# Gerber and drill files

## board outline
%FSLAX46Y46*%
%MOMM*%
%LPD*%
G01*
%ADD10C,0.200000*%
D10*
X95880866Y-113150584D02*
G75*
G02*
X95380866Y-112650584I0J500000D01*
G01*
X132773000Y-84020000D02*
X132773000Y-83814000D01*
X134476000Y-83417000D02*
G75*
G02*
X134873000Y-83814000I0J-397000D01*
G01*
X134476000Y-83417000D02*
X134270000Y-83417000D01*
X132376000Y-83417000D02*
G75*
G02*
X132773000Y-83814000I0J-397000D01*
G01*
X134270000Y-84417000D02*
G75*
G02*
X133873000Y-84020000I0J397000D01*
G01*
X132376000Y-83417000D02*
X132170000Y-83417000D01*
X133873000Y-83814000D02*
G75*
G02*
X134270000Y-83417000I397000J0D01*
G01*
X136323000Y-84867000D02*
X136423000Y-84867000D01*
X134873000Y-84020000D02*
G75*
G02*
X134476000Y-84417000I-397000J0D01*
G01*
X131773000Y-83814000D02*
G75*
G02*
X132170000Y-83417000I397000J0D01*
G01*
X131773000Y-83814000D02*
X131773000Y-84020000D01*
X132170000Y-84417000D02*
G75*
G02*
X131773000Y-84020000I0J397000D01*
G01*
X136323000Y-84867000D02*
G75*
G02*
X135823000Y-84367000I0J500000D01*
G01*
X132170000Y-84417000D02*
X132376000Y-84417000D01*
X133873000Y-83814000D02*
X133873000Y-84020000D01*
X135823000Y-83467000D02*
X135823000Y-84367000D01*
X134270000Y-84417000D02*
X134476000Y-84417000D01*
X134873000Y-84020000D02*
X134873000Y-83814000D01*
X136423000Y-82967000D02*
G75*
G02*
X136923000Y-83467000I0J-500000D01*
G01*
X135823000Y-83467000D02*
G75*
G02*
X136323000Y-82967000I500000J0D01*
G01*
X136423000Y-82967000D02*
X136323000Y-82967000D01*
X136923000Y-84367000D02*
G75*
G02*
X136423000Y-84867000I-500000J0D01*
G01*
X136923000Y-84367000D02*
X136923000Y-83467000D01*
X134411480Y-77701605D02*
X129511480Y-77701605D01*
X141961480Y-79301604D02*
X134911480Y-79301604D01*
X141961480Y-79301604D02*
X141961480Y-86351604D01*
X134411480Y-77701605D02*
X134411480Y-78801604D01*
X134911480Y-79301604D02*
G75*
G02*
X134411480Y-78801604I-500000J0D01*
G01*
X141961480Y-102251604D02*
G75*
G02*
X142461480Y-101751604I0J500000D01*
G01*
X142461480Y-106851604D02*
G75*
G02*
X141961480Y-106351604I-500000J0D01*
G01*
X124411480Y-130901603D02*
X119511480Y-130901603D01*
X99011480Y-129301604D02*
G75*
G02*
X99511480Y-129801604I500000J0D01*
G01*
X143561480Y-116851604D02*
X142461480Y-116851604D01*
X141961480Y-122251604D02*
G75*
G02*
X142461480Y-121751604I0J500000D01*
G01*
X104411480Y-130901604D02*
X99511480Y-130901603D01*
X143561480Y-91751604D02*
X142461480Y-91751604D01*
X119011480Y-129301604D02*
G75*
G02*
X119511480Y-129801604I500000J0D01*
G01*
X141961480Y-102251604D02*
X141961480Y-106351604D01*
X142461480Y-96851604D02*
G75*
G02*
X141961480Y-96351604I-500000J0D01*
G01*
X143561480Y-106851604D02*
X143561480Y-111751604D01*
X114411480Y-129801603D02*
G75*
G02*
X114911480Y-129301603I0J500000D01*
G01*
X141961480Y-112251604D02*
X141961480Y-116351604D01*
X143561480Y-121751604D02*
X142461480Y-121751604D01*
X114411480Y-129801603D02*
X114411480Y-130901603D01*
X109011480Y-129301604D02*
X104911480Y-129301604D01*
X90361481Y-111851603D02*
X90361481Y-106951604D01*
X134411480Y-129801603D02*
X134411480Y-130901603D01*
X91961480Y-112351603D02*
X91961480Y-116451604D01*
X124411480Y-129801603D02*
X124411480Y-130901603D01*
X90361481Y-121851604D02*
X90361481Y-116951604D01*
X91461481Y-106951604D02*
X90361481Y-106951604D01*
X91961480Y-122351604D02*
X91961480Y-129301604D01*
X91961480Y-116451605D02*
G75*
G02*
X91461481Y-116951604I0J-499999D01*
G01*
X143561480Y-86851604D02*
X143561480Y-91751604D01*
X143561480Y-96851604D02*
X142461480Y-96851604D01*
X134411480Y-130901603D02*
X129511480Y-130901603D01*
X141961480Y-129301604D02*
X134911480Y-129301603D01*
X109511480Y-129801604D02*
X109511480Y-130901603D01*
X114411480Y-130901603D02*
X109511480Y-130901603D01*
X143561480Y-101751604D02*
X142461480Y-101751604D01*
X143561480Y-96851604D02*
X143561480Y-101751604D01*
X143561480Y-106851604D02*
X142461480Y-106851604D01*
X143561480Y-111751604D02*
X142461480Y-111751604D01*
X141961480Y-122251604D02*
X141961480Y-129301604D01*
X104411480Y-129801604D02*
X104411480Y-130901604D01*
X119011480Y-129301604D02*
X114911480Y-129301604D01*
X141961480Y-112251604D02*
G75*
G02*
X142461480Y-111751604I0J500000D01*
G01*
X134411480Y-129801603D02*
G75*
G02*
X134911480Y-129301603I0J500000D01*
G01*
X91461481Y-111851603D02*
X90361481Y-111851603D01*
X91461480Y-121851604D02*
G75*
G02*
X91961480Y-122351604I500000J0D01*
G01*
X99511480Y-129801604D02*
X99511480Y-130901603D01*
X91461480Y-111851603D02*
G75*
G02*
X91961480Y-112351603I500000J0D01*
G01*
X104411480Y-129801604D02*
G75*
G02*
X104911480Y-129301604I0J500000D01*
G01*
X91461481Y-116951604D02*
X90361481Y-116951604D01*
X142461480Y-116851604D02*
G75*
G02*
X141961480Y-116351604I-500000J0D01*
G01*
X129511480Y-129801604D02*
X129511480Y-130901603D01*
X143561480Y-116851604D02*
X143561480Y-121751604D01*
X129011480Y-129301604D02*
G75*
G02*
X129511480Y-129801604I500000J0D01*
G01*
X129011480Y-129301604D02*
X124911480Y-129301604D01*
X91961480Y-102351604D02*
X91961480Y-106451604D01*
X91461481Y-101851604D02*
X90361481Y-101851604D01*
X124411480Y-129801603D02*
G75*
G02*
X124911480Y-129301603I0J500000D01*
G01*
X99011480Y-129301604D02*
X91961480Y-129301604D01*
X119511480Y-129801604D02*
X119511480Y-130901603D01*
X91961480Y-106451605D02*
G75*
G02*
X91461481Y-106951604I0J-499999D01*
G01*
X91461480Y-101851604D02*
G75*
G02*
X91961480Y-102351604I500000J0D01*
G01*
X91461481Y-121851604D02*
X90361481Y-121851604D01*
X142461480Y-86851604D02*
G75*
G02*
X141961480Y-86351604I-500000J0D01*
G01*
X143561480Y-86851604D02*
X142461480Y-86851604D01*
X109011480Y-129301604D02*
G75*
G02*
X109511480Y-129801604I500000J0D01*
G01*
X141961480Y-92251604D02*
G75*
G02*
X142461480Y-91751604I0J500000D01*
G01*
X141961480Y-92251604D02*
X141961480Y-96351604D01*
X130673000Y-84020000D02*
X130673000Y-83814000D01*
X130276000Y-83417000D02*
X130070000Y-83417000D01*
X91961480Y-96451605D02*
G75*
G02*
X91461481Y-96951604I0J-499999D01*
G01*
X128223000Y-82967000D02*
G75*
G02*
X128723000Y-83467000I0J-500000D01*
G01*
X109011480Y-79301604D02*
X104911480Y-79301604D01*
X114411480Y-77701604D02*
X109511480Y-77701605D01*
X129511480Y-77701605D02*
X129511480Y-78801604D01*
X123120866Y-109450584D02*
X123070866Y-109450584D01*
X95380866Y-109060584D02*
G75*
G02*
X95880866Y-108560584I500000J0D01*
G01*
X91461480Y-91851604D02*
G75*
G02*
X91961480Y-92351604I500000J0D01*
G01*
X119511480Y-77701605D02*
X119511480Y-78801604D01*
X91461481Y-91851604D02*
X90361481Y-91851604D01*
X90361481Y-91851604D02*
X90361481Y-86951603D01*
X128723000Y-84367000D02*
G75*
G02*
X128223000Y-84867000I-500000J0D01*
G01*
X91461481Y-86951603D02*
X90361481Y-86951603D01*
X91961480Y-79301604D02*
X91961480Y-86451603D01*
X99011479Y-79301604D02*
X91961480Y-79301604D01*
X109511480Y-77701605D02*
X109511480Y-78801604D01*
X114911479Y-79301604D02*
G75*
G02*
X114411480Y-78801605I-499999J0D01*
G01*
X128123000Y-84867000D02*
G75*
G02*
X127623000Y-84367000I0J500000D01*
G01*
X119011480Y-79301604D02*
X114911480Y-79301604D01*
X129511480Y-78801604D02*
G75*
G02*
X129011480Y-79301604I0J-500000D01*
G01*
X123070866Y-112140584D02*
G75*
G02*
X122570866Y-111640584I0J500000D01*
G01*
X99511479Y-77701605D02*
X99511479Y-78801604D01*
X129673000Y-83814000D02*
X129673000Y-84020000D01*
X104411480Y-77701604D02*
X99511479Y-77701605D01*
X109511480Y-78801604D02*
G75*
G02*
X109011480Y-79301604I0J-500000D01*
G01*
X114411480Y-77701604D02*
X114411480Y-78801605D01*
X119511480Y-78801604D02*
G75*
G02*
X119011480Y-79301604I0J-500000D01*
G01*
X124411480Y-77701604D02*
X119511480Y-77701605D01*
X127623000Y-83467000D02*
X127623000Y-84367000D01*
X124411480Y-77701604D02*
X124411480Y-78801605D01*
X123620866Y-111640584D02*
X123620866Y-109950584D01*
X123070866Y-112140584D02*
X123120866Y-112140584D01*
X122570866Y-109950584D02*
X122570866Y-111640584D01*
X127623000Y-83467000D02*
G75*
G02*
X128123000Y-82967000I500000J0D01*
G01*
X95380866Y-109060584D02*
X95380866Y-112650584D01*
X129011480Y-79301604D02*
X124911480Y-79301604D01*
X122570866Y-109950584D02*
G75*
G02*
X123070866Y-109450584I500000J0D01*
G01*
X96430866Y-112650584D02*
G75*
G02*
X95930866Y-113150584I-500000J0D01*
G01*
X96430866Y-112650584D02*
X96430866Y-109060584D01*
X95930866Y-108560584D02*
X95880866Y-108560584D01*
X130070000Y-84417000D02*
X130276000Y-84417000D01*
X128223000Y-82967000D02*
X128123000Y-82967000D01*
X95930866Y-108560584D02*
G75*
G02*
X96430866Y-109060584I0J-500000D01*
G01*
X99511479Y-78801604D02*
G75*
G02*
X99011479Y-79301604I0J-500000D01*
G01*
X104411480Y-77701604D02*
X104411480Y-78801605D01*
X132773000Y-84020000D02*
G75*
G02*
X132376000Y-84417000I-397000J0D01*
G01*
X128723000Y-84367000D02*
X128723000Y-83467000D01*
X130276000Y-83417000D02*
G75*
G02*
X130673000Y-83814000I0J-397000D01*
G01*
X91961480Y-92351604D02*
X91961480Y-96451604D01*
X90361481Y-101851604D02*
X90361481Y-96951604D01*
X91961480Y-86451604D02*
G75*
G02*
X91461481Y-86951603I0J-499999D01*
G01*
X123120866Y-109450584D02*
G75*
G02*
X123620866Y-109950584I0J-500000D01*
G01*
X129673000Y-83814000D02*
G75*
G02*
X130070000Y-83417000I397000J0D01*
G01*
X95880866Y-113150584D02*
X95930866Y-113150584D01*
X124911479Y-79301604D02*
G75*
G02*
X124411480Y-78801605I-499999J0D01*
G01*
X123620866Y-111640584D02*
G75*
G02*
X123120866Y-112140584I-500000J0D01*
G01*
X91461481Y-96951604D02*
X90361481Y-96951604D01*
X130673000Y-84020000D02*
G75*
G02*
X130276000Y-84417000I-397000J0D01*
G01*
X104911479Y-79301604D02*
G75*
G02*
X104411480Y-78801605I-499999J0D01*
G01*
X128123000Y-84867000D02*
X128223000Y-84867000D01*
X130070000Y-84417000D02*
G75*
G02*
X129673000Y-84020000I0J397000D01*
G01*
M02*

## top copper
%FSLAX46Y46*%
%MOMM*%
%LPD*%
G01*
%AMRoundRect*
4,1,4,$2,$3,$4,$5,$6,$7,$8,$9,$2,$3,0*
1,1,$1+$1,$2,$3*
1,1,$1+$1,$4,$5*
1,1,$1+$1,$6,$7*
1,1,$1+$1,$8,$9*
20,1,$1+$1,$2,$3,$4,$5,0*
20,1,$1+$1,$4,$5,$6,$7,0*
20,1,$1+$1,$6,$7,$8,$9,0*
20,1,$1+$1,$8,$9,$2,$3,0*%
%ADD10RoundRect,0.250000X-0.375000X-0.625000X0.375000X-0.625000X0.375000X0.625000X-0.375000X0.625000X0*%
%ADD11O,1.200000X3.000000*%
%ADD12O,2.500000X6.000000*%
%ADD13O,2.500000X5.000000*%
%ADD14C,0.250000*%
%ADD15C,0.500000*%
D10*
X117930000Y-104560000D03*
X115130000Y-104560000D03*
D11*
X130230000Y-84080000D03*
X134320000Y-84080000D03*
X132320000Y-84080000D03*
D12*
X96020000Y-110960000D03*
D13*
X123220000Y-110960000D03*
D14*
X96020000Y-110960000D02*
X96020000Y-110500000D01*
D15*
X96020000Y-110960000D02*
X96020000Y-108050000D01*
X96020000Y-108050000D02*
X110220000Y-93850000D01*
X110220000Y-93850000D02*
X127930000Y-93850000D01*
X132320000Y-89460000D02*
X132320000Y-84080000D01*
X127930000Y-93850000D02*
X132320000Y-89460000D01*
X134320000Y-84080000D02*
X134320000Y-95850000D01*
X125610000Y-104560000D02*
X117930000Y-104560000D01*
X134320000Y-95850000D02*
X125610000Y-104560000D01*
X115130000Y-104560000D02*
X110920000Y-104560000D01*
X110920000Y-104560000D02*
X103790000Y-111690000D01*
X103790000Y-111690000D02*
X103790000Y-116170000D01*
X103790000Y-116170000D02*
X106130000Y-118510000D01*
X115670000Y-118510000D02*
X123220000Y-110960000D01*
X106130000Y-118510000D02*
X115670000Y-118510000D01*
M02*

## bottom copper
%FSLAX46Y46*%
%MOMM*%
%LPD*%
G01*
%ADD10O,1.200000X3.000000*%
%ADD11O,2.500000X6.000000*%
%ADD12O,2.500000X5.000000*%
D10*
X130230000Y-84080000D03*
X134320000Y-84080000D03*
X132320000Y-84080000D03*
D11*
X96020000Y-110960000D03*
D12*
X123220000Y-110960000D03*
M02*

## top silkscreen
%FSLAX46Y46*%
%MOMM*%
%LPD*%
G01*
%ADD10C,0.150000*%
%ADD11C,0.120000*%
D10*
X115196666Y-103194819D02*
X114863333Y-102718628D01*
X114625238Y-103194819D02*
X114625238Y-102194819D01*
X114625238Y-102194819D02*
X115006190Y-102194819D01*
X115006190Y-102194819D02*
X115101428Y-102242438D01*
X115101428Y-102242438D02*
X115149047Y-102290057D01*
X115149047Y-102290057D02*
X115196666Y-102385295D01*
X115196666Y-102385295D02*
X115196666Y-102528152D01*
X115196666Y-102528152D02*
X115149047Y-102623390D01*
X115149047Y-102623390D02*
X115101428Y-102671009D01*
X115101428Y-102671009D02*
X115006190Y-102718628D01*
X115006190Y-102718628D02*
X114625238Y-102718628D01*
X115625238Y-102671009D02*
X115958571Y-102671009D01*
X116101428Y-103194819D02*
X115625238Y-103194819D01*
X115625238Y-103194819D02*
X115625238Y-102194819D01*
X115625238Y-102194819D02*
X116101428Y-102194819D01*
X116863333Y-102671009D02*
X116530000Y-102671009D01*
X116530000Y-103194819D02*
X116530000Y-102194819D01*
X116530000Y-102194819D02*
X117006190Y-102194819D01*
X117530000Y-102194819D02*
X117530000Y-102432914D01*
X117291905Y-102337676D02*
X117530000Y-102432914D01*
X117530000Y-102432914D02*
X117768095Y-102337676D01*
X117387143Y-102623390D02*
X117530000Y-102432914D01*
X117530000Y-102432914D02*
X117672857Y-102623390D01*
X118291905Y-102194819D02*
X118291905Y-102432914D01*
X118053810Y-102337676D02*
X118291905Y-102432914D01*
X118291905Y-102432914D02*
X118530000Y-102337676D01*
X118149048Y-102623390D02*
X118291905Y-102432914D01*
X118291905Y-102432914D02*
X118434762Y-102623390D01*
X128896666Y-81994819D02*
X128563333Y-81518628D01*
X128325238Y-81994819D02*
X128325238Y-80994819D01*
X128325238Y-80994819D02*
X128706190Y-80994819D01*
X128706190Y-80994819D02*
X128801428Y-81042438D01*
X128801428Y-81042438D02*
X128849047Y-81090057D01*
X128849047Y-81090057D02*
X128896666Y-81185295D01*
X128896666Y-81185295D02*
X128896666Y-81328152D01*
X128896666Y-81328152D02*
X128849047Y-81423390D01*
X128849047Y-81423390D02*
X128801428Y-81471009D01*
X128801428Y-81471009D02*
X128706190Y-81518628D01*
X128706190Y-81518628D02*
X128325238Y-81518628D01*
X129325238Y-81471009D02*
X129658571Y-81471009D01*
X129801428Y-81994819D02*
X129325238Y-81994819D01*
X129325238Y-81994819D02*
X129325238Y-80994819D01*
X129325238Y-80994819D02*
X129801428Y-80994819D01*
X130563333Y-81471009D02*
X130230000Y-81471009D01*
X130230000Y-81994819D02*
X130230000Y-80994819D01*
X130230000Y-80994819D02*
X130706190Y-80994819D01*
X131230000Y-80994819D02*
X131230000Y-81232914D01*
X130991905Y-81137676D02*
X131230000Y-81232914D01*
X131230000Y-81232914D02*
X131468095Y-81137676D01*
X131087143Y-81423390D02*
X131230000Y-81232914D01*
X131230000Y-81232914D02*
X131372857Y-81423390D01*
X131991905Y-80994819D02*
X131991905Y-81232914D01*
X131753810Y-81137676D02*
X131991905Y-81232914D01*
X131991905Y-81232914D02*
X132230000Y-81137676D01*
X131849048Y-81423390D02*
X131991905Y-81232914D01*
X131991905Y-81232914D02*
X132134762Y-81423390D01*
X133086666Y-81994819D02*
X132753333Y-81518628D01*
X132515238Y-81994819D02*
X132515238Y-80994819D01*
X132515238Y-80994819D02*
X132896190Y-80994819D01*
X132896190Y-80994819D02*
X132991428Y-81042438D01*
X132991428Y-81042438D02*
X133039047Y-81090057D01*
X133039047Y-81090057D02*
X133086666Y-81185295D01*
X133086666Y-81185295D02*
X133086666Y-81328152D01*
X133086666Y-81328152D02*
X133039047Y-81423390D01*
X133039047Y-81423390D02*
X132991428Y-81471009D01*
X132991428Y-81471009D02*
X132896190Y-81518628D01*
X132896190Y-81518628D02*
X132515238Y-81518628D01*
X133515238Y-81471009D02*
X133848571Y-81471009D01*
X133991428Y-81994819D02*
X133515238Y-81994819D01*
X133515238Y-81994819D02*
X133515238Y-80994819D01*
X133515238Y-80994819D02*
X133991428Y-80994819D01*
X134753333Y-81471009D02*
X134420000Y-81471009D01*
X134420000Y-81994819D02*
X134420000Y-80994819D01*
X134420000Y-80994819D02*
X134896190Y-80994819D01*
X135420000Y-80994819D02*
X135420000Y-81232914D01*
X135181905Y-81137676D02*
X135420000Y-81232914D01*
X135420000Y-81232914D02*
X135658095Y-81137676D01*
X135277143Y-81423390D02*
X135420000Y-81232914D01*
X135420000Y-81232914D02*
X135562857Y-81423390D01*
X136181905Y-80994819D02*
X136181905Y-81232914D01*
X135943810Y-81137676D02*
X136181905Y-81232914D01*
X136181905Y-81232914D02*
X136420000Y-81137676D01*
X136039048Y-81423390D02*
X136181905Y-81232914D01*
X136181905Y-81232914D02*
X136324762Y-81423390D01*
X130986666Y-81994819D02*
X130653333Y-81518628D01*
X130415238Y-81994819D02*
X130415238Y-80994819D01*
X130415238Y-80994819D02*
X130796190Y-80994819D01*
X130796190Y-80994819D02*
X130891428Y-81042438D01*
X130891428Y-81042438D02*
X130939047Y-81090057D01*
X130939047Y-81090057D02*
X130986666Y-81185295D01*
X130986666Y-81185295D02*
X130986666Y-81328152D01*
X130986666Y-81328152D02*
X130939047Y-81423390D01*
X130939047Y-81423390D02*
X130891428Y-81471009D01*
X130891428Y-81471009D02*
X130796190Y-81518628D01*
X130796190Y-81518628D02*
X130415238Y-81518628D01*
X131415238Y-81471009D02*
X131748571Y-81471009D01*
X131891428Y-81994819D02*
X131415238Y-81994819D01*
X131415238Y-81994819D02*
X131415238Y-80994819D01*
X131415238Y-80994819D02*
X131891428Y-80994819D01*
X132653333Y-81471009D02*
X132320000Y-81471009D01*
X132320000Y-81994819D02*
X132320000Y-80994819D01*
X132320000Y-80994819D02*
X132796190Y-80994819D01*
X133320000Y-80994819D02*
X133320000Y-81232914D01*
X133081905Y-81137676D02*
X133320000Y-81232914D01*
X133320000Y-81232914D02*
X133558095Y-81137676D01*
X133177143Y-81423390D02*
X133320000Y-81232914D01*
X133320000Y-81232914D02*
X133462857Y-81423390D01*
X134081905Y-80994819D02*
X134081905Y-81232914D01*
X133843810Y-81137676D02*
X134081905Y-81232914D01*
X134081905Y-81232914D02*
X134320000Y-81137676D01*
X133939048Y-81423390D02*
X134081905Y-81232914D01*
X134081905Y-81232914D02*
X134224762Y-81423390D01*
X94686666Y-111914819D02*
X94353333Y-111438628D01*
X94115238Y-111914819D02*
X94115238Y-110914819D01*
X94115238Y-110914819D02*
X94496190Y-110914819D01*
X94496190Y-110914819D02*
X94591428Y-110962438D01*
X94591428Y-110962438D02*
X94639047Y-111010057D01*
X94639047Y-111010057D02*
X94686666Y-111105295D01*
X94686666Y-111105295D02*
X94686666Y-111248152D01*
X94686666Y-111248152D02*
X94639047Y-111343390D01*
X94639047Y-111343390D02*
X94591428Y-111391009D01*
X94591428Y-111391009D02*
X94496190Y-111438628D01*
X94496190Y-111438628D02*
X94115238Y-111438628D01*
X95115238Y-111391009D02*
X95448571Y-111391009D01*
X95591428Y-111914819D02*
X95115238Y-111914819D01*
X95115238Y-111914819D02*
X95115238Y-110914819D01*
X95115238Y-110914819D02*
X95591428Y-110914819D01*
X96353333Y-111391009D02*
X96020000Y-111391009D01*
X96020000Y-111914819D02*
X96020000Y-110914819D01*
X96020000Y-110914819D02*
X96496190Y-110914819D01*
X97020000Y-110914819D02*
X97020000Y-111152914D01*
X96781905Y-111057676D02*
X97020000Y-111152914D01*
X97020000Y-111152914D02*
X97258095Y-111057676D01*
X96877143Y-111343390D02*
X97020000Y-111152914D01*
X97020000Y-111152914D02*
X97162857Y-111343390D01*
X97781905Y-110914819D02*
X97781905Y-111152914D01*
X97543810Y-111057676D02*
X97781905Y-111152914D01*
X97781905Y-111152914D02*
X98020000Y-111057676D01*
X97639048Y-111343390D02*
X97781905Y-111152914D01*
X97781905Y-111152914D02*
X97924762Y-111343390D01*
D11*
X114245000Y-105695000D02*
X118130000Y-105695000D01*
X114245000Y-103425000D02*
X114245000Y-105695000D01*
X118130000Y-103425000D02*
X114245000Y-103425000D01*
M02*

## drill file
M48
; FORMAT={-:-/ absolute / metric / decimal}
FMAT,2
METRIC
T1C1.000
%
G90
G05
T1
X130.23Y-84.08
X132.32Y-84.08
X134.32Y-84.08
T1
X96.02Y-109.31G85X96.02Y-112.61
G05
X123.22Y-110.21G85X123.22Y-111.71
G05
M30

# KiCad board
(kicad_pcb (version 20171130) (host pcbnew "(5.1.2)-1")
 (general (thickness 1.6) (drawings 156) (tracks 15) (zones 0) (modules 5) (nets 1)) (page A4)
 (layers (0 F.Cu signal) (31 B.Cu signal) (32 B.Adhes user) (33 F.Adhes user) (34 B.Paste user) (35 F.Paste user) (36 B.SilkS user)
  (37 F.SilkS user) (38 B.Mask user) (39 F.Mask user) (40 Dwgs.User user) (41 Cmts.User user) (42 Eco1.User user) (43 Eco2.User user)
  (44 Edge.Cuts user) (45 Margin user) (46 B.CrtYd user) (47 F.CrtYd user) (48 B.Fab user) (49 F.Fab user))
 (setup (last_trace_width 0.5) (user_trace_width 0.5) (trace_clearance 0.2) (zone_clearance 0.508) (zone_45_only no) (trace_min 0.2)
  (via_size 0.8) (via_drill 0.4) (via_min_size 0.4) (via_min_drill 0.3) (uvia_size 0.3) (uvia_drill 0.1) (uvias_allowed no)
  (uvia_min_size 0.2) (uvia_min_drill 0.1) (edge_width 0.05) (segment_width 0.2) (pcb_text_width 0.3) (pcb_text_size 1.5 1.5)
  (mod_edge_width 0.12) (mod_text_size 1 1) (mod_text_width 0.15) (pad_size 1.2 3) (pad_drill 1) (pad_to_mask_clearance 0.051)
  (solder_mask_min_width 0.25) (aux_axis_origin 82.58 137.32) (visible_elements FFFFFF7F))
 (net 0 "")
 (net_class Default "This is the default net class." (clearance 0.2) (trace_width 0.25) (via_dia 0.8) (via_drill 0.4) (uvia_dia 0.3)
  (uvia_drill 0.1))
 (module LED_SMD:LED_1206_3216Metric (layer F.Cu) (at 116.53 104.56)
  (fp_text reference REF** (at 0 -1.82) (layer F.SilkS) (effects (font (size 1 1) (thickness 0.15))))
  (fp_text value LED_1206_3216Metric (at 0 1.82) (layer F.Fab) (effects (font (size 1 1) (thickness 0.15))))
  (fp_line (start -2.285 1.135) (end 1.6 1.135) (layer F.SilkS) (width 0.12))
  (fp_line (start -2.285 -1.135) (end -2.285 1.135) (layer F.SilkS) (width 0.12))
  (fp_line (start 1.6 -1.135) (end -2.285 -1.135) (layer F.SilkS) (width 0.12))
  (pad 2 smd roundrect (at 1.4 0) (size 1.25 1.75) (layers F.Cu F.Paste F.Mask) (roundrect_rratio 0.2))
  (pad 1 smd roundrect (at -1.4 0) (size 1.25 1.75) (layers F.Cu F.Paste F.Mask) (roundrect_rratio 0.2)))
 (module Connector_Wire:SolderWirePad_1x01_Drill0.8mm (layer F.Cu) (at 130.23 84.08)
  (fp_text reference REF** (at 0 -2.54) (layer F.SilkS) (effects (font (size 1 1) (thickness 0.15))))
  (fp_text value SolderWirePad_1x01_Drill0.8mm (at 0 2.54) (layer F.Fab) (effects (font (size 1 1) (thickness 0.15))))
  (pad 1 thru_hole oval (at 0 0) (size 1.2 3) (drill 1) (layers F.Cu)))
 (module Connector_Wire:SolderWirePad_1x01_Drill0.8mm (layer F.Cu) (at 134.42 84.08)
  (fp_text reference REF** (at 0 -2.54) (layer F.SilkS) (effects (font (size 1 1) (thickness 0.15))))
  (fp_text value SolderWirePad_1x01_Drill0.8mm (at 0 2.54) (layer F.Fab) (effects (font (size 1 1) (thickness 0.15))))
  (pad 1 thru_hole oval (at -0.1 0) (size 1.2 3) (drill 1) (layers F.Cu)))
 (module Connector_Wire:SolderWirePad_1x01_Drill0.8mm (layer F.Cu) (at 132.32 84.08)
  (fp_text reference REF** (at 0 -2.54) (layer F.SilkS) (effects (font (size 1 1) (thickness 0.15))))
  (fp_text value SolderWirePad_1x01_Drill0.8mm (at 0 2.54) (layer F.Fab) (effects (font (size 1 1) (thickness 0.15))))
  (pad 1 thru_hole oval (at 0 0) (size 1.2 3) (drill 1) (layers F.Cu)))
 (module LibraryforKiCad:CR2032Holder (layer F.Cu) (at 96.02 110.96)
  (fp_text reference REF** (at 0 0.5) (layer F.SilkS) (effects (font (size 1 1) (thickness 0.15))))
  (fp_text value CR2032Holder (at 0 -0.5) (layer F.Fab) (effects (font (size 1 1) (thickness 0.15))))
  (pad 2 thru_hole oval (at 0 0) (size 2.5 6) (drill oval 1 4.3) (layers F.Cu F.Adhes))
  (pad 1 thru_hole oval (at 27.2 0) (size 2.5 5) (drill oval 1 2.5) (layers F.Cu)))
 (gr_arc (start 95.880866 112.650584) (end 95.380866 112.650584) (angle -90) (layer Edge.Cuts) (width 0.2))
 (gr_line (start 132.773 84.02) (end 132.773 83.814) (layer Edge.Cuts) (width 0.2))
 (gr_arc (start 134.476 83.814) (end 134.873 83.814) (angle -90) (layer Edge.Cuts) (width 0.2))
 (gr_line (start 134.476 83.417) (end 134.27 83.417) (layer Edge.Cuts) (width 0.2))
 (gr_arc (start 132.376 83.814) (end 132.773 83.814) (angle -90) (layer Edge.Cuts) (width 0.2))
 (gr_arc (start 134.27 84.02) (end 133.873 84.02) (angle -90) (layer Edge.Cuts) (width 0.2))
 (gr_line (start 132.376 83.417) (end 132.17 83.417) (layer Edge.Cuts) (width 0.2))
 (gr_arc (start 134.27 83.814) (end 134.27 83.417) (angle -90) (layer Edge.Cuts) (width 0.2))
 (gr_line (start 136.323 84.867) (end 136.423 84.867) (layer Edge.Cuts) (width 0.2))
 (gr_arc (start 134.476 84.02) (end 134.476 84.417) (angle -90) (layer Edge.Cuts) (width 0.2))
 (gr_arc (start 132.17 83.814) (end 132.17 83.417) (angle -90) (layer Edge.Cuts) (width 0.2))
 (gr_line (start 131.773 83.814) (end 131.773 84.02) (layer Edge.Cuts) (width 0.2))
 (gr_arc (start 132.17 84.02) (end 131.773 84.02) (angle -90) (layer Edge.Cuts) (width 0.2))
 (gr_arc (start 136.323 84.367) (end 135.823 84.367) (angle -90) (layer Edge.Cuts) (width 0.2))
 (gr_line (start 132.17 84.417) (end 132.376 84.417) (layer Edge.Cuts) (width 0.2))
 (gr_line (start 133.873 83.814) (end 133.873 84.02) (layer Edge.Cuts) (width 0.2))
 (gr_line (start 135.823 83.467) (end 135.823 84.367) (layer Edge.Cuts) (width 0.2))
 (gr_line (start 134.27 84.417) (end 134.476 84.417) (layer Edge.Cuts) (width 0.2))
 (gr_line (start 134.873 84.02) (end 134.873 83.814) (layer Edge.Cuts) (width 0.2))
 (gr_arc (start 136.423 83.467) (end 136.923 83.467) (angle -90) (layer Edge.Cuts) (width 0.2))
 (gr_arc (start 136.323 83.467) (end 136.323 82.967) (angle -90) (layer Edge.Cuts) (width 0.2))
 (gr_line (start 136.423 82.967) (end 136.323 82.967) (layer Edge.Cuts) (width 0.2))
 (gr_arc (start 136.423 84.367) (end 136.423 84.867) (angle -90) (layer Edge.Cuts) (width 0.2))
 (gr_line (start 136.923 84.367) (end 136.923 83.467) (layer Edge.Cuts) (width 0.2))
 (gr_line (start 134.41148 77.701605) (end 129.51148 77.701605) (layer Edge.Cuts) (width 0.2))
 (gr_line (start 141.96148 79.301604) (end 134.91148 79.301604) (layer Edge.Cuts) (width 0.2))
 (gr_line (start 141.96148 79.301604) (end 141.96148 86.351604) (layer Edge.Cuts) (width 0.2))
 (gr_line (start 134.41148 77.701605) (end 134.41148 78.801604) (layer Edge.Cuts) (width 0.2))
 (gr_arc (start 134.41148 79.301604) (end 134.41148 78.801604) (angle -270) (layer Edge.Cuts) (width 0.2))
 (gr_arc (start 141.96148 101.751604) (end 142.46148 101.751604) (angle -270) (layer Edge.Cuts) (width 0.2))
 (gr_arc (start 141.96148 106.851604) (end 141.96148 106.351604) (angle -270) (layer Edge.Cuts) (width 0.2))
 (gr_line (start 124.41148 130.901603) (end 119.51148 130.901603) (layer Edge.Cuts) (width 0.2))
 (gr_arc (start 99.51148 129.301604) (end 99.51148 129.801604) (angle -270) (layer Edge.Cuts) (width 0.2))
 (gr_line (start 143.56148 116.851604) (end 142.46148 116.851604) (layer Edge.Cuts) (width 0.2))
 (gr_arc (start 141.96148 121.751604) (end 142.46148 121.751604) (angle -270) (layer Edge.Cuts) (width 0.2))
 (gr_line (start 104.41148 130.901604) (end 99.51148 130.901603) (layer Edge.Cuts) (width 0.2))
 (gr_line (start 143.56148 91.751604) (end 142.46148 91.751604) (layer Edge.Cuts) (width 0.2))
 (gr_arc (start 119.51148 129.301604) (end 119.51148 129.801604) (angle -270) (layer Edge.Cuts) (width 0.2))
 (gr_line (start 141.96148 102.251604) (end 141.96148 106.351604) (layer Edge.Cuts) (width 0.2))
 (gr_arc (start 141.96148 96.851604) (end 141.96148 96.351604) (angle -270) (layer Edge.Cuts) (width 0.2))
 (gr_line (start 143.56148 106.851604) (end 143.56148 111.751604) (layer Edge.Cuts) (width 0.2))
 (gr_arc (start 114.41148 129.301603) (end 114.91148 129.301603) (angle -270) (layer Edge.Cuts) (width 0.2))
 (gr_line (start 141.96148 112.251604) (end 141.96148 116.351604) (layer Edge.Cuts) (width 0.2))
 (gr_line (start 143.56148 121.751604) (end 142.46148 121.751604) (layer Edge.Cuts) (width 0.2))
 (gr_line (start 114.41148 129.801603) (end 114.41148 130.901603) (layer Edge.Cuts) (width 0.2))
 (gr_line (start 109.01148 129.301604) (end 104.91148 129.301604) (layer Edge.Cuts) (width 0.2))
 (gr_line (start 90.361481 111.851603) (end 90.361481 106.951604) (layer Edge.Cuts) (width 0.2))
 (gr_line (start 134.41148 129.801603) (end 134.41148 130.901603) (layer Edge.Cuts) (width 0.2))
 (gr_line (start 91.96148 112.351603) (end 91.96148 116.451604) (layer Edge.Cuts) (width 0.2))
 (gr_line (start 124.41148 129.801603) (end 124.41148 130.901603) (layer Edge.Cuts) (width 0.2))
 (gr_line (start 90.361481 121.851604) (end 90.361481 116.951604) (layer Edge.Cuts) (width 0.2))
 (gr_line (start 91.461481 106.951604) (end 90.361481 106.951604) (layer Edge.Cuts) (width 0.2))
 (gr_line (start 91.96148 122.351604) (end 91.96148 129.301604) (layer Edge.Cuts) (width 0.2))
 (gr_arc (start 91.96148 116.951604) (end 91.461481 116.951604) (angle -270) (layer Edge.Cuts) (width 0.2))
 (gr_line (start 143.56148 86.851604) (end 143.56148 91.751604) (layer Edge.Cuts) (width 0.2))
 (gr_line (start 143.56148 96.851604) (end 142.46148 96.851604) (layer Edge.Cuts) (width 0.2))
 (gr_line (start 134.41148 130.901603) (end 129.51148 130.901603) (layer Edge.Cuts) (width 0.2))
 (gr_line (start 141.96148 129.301604) (end 134.91148 129.301603) (layer Edge.Cuts) (width 0.2))
 (gr_line (start 109.51148 129.801604) (end 109.51148 130.901603) (layer Edge.Cuts) (width 0.2))
 (gr_line (start 114.41148 130.901603) (end 109.51148 130.901603) (layer Edge.Cuts) (width 0.2))
 (gr_line (start 143.56148 101.751604) (end 142.46148 101.751604) (layer Edge.Cuts) (width 0.2))
 (gr_line (start 143.56148 96.851604) (end 143.56148 101.751604) (layer Edge.Cuts) (width 0.2))
 (gr_line (start 143.56148 106.851604) (end 142.46148 106.851604) (layer Edge.Cuts) (width 0.2))
 (gr_line (start 143.56148 111.751604) (end 142.46148 111.751604) (layer Edge.Cuts) (width 0.2))
 (gr_line (start 141.96148 122.251604) (end 141.96148 129.301604) (layer Edge.Cuts) (width 0.2))
 (gr_line (start 104.41148 129.801604) (end 104.41148 130.901604) (layer Edge.Cuts) (width 0.2))
 (gr_line (start 119.01148 129.301604) (end 114.91148 129.301604) (layer Edge.Cuts) (width 0.2))
 (gr_arc (start 141.96148 111.751604) (end 142.46148 111.751604) (angle -270) (layer Edge.Cuts) (width 0.2))
 (gr_arc (start 134.41148 129.301603) (end 134.91148 129.301603) (angle -270) (layer Edge.Cuts) (width 0.2))
 (gr_line (start 91.461481 111.851603) (end 90.361481 111.851603) (layer Edge.Cuts) (width 0.2))
 (gr_arc (start 91.96148 121.851604) (end 91.96148 122.351604) (angle -270) (layer Edge.Cuts) (width 0.2))
 (gr_line (start 99.51148 129.801604) (end 99.51148 130.901603) (layer Edge.Cuts) (width 0.2))
 (gr_arc (start 91.96148 111.851603) (end 91.96148 112.351603) (angle -270) (layer Edge.Cuts) (width 0.2))
 (gr_arc (start 104.41148 129.301604) (end 104.91148 129.301604) (angle -270) (layer Edge.Cuts) (width 0.2))
 (gr_line (start 91.461481 116.951604) (end 90.361481 116.951604) (layer Edge.Cuts) (width 0.2))
 (gr_arc (start 141.96148 116.851604) (end 141.96148 116.351604) (angle -270) (layer Edge.Cuts) (width 0.2))
 (gr_line (start 129.51148 129.801604) (end 129.51148 130.901603) (layer Edge.Cuts) (width 0.2))
 (gr_line (start 143.56148 116.851604) (end 143.56148 121.751604) (layer Edge.Cuts) (width 0.2))
 (gr_arc (start 129.51148 129.301604) (end 129.51148 129.801604) (angle -270) (layer Edge.Cuts) (width 0.2))
 (gr_line (start 129.01148 129.301604) (end 124.91148 129.301604) (layer Edge.Cuts) (width 0.2))
 (gr_line (start 91.96148 102.351604) (end 91.96148 106.451604) (layer Edge.Cuts) (width 0.2))
 (gr_line (start 91.461481 101.851604) (end 90.361481 101.851604) (layer Edge.Cuts) (width 0.2))
 (gr_arc (start 124.41148 129.301603) (end 124.91148 129.301603) (angle -270) (layer Edge.Cuts) (width 0.2))
 (gr_line (start 99.01148 129.301604) (end 91.96148 129.301604) (layer Edge.Cuts) (width 0.2))
 (gr_line (start 119.51148 129.801604) (end 119.51148 130.901603) (layer Edge.Cuts) (width 0.2))
 (gr_arc (start 91.96148 106.951604) (end 91.461481 106.951604) (angle -270) (layer Edge.Cuts) (width 0.2))
 (gr_arc (start 91.96148 101.851604) (end 91.96148 102.351604) (angle -270) (layer Edge.Cuts) (width 0.2))
 (gr_line (start 91.461481 121.851604) (end 90.361481 121.851604) (layer Edge.Cuts) (width 0.2))
 (gr_arc (start 141.96148 86.851604) (end 141.96148 86.351604) (angle -270) (layer Edge.Cuts) (width 0.2))
 (gr_line (start 143.56148 86.851604) (end 142.46148 86.851604) (layer Edge.Cuts) (width 0.2))
 (gr_arc (start 109.51148 129.301604) (end 109.51148 129.801604) (angle -270) (layer Edge.Cuts) (width 0.2))
 (gr_arc (start 141.96148 91.751604) (end 142.46148 91.751604) (angle -270) (layer Edge.Cuts) (width 0.2))
 (gr_line (start 141.96148 92.251604) (end 141.96148 96.351604) (layer Edge.Cuts) (width 0.2))
 (gr_line (start 130.673 84.02) (end 130.673 83.814) (layer Edge.Cuts) (width 0.2))
 (gr_line (start 130.276 83.417) (end 130.07 83.417) (layer Edge.Cuts) (width 0.2))
 (gr_arc (start 91.96148 96.951604) (end 91.461481 96.951604) (angle -270) (layer Edge.Cuts) (width 0.2))
 (gr_arc (start 128.223 83.467) (end 128.723 83.467) (angle -90) (layer Edge.Cuts) (width 0.2))
 (gr_line (start 109.01148 79.301604) (end 104.91148 79.301604) (layer Edge.Cuts) (width 0.2))
 (gr_line (start 114.41148 77.701604) (end 109.51148 77.701605) (layer Edge.Cuts) (width 0.2))
 (gr_line (start 129.51148 77.701605) (end 129.51148 78.801604) (layer Edge.Cuts) (width 0.2))
 (gr_line (start 123.120866 109.450584) (end 123.070866 109.450584) (layer Edge.Cuts) (width 0.2))
 (gr_arc (start 95.880866 109.060584) (end 95.880866 108.560584) (angle -90) (layer Edge.Cuts) (width 0.2))
 (gr_arc (start 91.96148 91.851604) (end 91.96148 92.351604) (angle -270) (layer Edge.Cuts) (width 0.2))
 (gr_line (start 119.51148 77.701605) (end 119.51148 78.801604) (layer Edge.Cuts) (width 0.2))
 (gr_line (start 91.461481 91.851604) (end 90.361481 91.851604) (layer Edge.Cuts) (width 0.2))
 (gr_line (start 90.361481 91.851604) (end 90.361481 86.951603) (layer Edge.Cuts) (width 0.2))
 (gr_arc (start 128.223 84.367) (end 128.223 84.867) (angle -90) (layer Edge.Cuts) (width 0.2))
 (gr_line (start 91.461481 86.951603) (end 90.361481 86.951603) (layer Edge.Cuts) (width 0.2))
 (gr_line (start 91.96148 79.301604) (end 91.96148 86.451603) (layer Edge.Cuts) (width 0.2))
 (gr_line (start 99.011479 79.301604) (end 91.96148 79.301604) (layer Edge.Cuts) (width 0.2))
 (gr_line (start 109.51148 77.701605) (end 109.51148 78.801604) (layer Edge.Cuts) (width 0.2))
 (gr_arc (start 114.41148 79.301604) (end 114.41148 78.801605) (angle -270) (layer Edge.Cuts) (width 0.2))
 (gr_arc (start 128.123 84.367) (end 127.623 84.367) (angle -90) (layer Edge.Cuts) (width 0.2))
 (gr_line (start 119.01148 79.301604) (end 114.91148 79.301604) (layer Edge.Cuts) (width 0.2))
 (gr_arc (start 129.51148 79.301604) (end 129.01148 79.301604) (angle -270) (layer Edge.Cuts) (width 0.2))
 (gr_arc (start 123.070866 111.640584) (end 122.570866 111.640584) (angle -90) (layer Edge.Cuts) (width 0.2))
 (gr_line (start 99.511479 77.701605) (end 99.511479 78.801604) (layer Edge.Cuts) (width 0.2))
 (gr_line (start 129.673 83.814) (end 129.673 84.02) (layer Edge.Cuts) (width 0.2))
 (gr_line (start 104.41148 77.701604) (end 99.511479 77.701605) (layer Edge.Cuts) (width 0.2))
 (gr_arc (start 109.51148 79.301604) (end 109.01148 79.301604) (angle -270) (layer Edge.Cuts) (width 0.2))
 (gr_line (start 114.41148 77.701604) (end 114.41148 78.801605) (layer Edge.Cuts) (width 0.2))
 (gr_arc (start 119.51148 79.301604) (end 119.01148 79.301604) (angle -270) (layer Edge.Cuts) (width 0.2))
 (gr_line (start 124.41148 77.701604) (end 119.51148 77.701605) (layer Edge.Cuts) (width 0.2))
 (gr_line (start 127.623 83.467) (end 127.623 84.367) (layer Edge.Cuts) (width 0.2))
 (gr_line (start 124.41148 77.701604) (end 124.41148 78.801605) (layer Edge.Cuts) (width 0.2))
 (gr_line (start 123.620866 111.640584) (end 123.620866 109.950584) (layer Edge.Cuts) (width 0.2))
 (gr_line (start 123.070866 112.140584) (end 123.120866 112.140584) (layer Edge.Cuts) (width 0.2))
 (gr_line (start 122.570866 109.950584) (end 122.570866 111.640584) (layer Edge.Cuts) (width 0.2))
 (gr_arc (start 128.123 83.467) (end 128.123 82.967) (angle -90) (layer Edge.Cuts) (width 0.2))
 (gr_line (start 95.380866 109.060584) (end 95.380866 112.650584) (layer Edge.Cuts) (width 0.2))
 (gr_line (start 129.01148 79.301604) (end 124.91148 79.301604) (layer Edge.Cuts) (width 0.2))
 (gr_arc (start 123.070866 109.950584) (end 123.070866 109.450584) (angle -90) (layer Edge.Cuts) (width 0.2))
 (gr_arc (start 95.930866 112.650584) (end 95.930866 113.150584) (angle -90) (layer Edge.Cuts) (width 0.2))
 (gr_line (start 96.430866 112.650584) (end 96.430866 109.060584) (layer Edge.Cuts) (width 0.2))
 (gr_line (start 95.930866 108.560584) (end 95.880866 108.560584) (layer Edge.Cuts) (width 0.2))
 (gr_line (start 130.07 84.417) (end 130.276 84.417) (layer Edge.Cuts) (width 0.2))
 (gr_line (start 128.223 82.967) (end 128.123 82.967) (layer Edge.Cuts) (width 0.2))
 (gr_arc (start 95.930866 109.060584) (end 96.430866 109.060584) (angle -90) (layer Edge.Cuts) (width 0.2))
 (gr_arc (start 99.511479 79.301604) (end 99.011479 79.301604) (angle -270) (layer Edge.Cuts) (width 0.2))
 (gr_line (start 104.41148 77.701604) (end 104.41148 78.801605) (layer Edge.Cuts) (width 0.2))
 (gr_arc (start 132.376 84.02) (end 132.376 84.417) (angle -90) (layer Edge.Cuts) (width 0.2))
 (gr_line (start 128.723 84.367) (end 128.723 83.467) (layer Edge.Cuts) (width 0.2))
 (gr_arc (start 130.276 83.814) (end 130.673 83.814) (angle -90) (layer Edge.Cuts) (width 0.2))
 (gr_line (start 91.96148 92.351604) (end 91.96148 96.451604) (layer Edge.Cuts) (width 0.2))
 (gr_line (start 90.361481 101.851604) (end 90.361481 96.951604) (layer Edge.Cuts) (width 0.2))
 (gr_arc (start 91.96148 86.951603) (end 91.461481 86.951603) (angle -270) (layer Edge.Cuts) (width 0.2))
 (gr_arc (start 123.120866 109.950584) (end 123.620866 109.950584) (angle -90) (layer Edge.Cuts) (width 0.2))
 (gr_arc (start 130.07 83.814) (end 130.07 83.417) (angle -90) (layer Edge.Cuts) (width 0.2))
 (gr_line (start 95.880866 113.150584) (end 95.930866 113.150584) (layer Edge.Cuts) (width 0.2))
 (gr_arc (start 124.41148 79.301604) (end 124.41148 78.801605) (angle -270) (layer Edge.Cuts) (width 0.2))
 (gr_arc (start 123.120866 111.640584) (end 123.120866 112.140584) (angle -90) (layer Edge.Cuts) (width 0.2))
 (gr_line (start 91.461481 96.951604) (end 90.361481 96.951604) (layer Edge.Cuts) (width 0.2))
 (gr_arc (start 130.276 84.02) (end 130.276 84.417) (angle -90) (layer Edge.Cuts) (width 0.2))
 (gr_arc (start 104.41148 79.301604) (end 104.41148 78.801605) (angle -270) (layer Edge.Cuts) (width 0.2))
 (gr_line (start 128.123 84.867) (end 128.223 84.867) (layer Edge.Cuts) (width 0.2))
 (gr_arc (start 130.07 84.02) (end 129.673 84.02) (angle -90) (layer Edge.Cuts) (width 0.2))
 (segment (start 96.02 110.96) (end 96.02 110.5) (width 0.25) (layer F.Cu) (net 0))
 (segment (start 96.02 110.96) (end 96.02 108.05) (width 0.5) (layer F.Cu) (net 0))
 (segment (start 96.02 108.05) (end 110.22 93.85) (width 0.5) (layer F.Cu) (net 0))
 (segment (start 110.22 93.85) (end 127.93 93.85) (width 0.5) (layer F.Cu) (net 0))
 (segment (start 132.32 89.46) (end 132.32 84.08) (width 0.5) (layer F.Cu) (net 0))
 (segment (start 127.93 93.85) (end 132.32 89.46) (width 0.5) (layer F.Cu) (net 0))
 (segment (start 134.32 84.08) (end 134.32 95.85) (width 0.5) (layer F.Cu) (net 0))
 (segment (start 125.61 104.56) (end 117.93 104.56) (width 0.5) (layer F.Cu) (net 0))
 (segment (start 134.32 95.85) (end 125.61 104.56) (width 0.5) (layer F.Cu) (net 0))
 (segment (start 115.13 104.56) (end 110.92 104.56) (width 0.5) (layer F.Cu) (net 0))
 (segment (start 110.92 104.56) (end 103.79 111.69) (width 0.5) (layer F.Cu) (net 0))
 (segment (start 103.79 111.69) (end 103.79 116.17) (width 0.5) (layer F.Cu) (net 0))
 (segment (start 103.79 116.17) (end 106.13 118.51) (width 0.5) (layer F.Cu) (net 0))
 (segment (start 115.67 118.51) (end 123.22 110.96) (width 0.5) (layer F.Cu) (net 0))
 (segment (start 106.13 118.51) (end 115.67 118.51) (width 0.5) (layer F.Cu) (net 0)))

